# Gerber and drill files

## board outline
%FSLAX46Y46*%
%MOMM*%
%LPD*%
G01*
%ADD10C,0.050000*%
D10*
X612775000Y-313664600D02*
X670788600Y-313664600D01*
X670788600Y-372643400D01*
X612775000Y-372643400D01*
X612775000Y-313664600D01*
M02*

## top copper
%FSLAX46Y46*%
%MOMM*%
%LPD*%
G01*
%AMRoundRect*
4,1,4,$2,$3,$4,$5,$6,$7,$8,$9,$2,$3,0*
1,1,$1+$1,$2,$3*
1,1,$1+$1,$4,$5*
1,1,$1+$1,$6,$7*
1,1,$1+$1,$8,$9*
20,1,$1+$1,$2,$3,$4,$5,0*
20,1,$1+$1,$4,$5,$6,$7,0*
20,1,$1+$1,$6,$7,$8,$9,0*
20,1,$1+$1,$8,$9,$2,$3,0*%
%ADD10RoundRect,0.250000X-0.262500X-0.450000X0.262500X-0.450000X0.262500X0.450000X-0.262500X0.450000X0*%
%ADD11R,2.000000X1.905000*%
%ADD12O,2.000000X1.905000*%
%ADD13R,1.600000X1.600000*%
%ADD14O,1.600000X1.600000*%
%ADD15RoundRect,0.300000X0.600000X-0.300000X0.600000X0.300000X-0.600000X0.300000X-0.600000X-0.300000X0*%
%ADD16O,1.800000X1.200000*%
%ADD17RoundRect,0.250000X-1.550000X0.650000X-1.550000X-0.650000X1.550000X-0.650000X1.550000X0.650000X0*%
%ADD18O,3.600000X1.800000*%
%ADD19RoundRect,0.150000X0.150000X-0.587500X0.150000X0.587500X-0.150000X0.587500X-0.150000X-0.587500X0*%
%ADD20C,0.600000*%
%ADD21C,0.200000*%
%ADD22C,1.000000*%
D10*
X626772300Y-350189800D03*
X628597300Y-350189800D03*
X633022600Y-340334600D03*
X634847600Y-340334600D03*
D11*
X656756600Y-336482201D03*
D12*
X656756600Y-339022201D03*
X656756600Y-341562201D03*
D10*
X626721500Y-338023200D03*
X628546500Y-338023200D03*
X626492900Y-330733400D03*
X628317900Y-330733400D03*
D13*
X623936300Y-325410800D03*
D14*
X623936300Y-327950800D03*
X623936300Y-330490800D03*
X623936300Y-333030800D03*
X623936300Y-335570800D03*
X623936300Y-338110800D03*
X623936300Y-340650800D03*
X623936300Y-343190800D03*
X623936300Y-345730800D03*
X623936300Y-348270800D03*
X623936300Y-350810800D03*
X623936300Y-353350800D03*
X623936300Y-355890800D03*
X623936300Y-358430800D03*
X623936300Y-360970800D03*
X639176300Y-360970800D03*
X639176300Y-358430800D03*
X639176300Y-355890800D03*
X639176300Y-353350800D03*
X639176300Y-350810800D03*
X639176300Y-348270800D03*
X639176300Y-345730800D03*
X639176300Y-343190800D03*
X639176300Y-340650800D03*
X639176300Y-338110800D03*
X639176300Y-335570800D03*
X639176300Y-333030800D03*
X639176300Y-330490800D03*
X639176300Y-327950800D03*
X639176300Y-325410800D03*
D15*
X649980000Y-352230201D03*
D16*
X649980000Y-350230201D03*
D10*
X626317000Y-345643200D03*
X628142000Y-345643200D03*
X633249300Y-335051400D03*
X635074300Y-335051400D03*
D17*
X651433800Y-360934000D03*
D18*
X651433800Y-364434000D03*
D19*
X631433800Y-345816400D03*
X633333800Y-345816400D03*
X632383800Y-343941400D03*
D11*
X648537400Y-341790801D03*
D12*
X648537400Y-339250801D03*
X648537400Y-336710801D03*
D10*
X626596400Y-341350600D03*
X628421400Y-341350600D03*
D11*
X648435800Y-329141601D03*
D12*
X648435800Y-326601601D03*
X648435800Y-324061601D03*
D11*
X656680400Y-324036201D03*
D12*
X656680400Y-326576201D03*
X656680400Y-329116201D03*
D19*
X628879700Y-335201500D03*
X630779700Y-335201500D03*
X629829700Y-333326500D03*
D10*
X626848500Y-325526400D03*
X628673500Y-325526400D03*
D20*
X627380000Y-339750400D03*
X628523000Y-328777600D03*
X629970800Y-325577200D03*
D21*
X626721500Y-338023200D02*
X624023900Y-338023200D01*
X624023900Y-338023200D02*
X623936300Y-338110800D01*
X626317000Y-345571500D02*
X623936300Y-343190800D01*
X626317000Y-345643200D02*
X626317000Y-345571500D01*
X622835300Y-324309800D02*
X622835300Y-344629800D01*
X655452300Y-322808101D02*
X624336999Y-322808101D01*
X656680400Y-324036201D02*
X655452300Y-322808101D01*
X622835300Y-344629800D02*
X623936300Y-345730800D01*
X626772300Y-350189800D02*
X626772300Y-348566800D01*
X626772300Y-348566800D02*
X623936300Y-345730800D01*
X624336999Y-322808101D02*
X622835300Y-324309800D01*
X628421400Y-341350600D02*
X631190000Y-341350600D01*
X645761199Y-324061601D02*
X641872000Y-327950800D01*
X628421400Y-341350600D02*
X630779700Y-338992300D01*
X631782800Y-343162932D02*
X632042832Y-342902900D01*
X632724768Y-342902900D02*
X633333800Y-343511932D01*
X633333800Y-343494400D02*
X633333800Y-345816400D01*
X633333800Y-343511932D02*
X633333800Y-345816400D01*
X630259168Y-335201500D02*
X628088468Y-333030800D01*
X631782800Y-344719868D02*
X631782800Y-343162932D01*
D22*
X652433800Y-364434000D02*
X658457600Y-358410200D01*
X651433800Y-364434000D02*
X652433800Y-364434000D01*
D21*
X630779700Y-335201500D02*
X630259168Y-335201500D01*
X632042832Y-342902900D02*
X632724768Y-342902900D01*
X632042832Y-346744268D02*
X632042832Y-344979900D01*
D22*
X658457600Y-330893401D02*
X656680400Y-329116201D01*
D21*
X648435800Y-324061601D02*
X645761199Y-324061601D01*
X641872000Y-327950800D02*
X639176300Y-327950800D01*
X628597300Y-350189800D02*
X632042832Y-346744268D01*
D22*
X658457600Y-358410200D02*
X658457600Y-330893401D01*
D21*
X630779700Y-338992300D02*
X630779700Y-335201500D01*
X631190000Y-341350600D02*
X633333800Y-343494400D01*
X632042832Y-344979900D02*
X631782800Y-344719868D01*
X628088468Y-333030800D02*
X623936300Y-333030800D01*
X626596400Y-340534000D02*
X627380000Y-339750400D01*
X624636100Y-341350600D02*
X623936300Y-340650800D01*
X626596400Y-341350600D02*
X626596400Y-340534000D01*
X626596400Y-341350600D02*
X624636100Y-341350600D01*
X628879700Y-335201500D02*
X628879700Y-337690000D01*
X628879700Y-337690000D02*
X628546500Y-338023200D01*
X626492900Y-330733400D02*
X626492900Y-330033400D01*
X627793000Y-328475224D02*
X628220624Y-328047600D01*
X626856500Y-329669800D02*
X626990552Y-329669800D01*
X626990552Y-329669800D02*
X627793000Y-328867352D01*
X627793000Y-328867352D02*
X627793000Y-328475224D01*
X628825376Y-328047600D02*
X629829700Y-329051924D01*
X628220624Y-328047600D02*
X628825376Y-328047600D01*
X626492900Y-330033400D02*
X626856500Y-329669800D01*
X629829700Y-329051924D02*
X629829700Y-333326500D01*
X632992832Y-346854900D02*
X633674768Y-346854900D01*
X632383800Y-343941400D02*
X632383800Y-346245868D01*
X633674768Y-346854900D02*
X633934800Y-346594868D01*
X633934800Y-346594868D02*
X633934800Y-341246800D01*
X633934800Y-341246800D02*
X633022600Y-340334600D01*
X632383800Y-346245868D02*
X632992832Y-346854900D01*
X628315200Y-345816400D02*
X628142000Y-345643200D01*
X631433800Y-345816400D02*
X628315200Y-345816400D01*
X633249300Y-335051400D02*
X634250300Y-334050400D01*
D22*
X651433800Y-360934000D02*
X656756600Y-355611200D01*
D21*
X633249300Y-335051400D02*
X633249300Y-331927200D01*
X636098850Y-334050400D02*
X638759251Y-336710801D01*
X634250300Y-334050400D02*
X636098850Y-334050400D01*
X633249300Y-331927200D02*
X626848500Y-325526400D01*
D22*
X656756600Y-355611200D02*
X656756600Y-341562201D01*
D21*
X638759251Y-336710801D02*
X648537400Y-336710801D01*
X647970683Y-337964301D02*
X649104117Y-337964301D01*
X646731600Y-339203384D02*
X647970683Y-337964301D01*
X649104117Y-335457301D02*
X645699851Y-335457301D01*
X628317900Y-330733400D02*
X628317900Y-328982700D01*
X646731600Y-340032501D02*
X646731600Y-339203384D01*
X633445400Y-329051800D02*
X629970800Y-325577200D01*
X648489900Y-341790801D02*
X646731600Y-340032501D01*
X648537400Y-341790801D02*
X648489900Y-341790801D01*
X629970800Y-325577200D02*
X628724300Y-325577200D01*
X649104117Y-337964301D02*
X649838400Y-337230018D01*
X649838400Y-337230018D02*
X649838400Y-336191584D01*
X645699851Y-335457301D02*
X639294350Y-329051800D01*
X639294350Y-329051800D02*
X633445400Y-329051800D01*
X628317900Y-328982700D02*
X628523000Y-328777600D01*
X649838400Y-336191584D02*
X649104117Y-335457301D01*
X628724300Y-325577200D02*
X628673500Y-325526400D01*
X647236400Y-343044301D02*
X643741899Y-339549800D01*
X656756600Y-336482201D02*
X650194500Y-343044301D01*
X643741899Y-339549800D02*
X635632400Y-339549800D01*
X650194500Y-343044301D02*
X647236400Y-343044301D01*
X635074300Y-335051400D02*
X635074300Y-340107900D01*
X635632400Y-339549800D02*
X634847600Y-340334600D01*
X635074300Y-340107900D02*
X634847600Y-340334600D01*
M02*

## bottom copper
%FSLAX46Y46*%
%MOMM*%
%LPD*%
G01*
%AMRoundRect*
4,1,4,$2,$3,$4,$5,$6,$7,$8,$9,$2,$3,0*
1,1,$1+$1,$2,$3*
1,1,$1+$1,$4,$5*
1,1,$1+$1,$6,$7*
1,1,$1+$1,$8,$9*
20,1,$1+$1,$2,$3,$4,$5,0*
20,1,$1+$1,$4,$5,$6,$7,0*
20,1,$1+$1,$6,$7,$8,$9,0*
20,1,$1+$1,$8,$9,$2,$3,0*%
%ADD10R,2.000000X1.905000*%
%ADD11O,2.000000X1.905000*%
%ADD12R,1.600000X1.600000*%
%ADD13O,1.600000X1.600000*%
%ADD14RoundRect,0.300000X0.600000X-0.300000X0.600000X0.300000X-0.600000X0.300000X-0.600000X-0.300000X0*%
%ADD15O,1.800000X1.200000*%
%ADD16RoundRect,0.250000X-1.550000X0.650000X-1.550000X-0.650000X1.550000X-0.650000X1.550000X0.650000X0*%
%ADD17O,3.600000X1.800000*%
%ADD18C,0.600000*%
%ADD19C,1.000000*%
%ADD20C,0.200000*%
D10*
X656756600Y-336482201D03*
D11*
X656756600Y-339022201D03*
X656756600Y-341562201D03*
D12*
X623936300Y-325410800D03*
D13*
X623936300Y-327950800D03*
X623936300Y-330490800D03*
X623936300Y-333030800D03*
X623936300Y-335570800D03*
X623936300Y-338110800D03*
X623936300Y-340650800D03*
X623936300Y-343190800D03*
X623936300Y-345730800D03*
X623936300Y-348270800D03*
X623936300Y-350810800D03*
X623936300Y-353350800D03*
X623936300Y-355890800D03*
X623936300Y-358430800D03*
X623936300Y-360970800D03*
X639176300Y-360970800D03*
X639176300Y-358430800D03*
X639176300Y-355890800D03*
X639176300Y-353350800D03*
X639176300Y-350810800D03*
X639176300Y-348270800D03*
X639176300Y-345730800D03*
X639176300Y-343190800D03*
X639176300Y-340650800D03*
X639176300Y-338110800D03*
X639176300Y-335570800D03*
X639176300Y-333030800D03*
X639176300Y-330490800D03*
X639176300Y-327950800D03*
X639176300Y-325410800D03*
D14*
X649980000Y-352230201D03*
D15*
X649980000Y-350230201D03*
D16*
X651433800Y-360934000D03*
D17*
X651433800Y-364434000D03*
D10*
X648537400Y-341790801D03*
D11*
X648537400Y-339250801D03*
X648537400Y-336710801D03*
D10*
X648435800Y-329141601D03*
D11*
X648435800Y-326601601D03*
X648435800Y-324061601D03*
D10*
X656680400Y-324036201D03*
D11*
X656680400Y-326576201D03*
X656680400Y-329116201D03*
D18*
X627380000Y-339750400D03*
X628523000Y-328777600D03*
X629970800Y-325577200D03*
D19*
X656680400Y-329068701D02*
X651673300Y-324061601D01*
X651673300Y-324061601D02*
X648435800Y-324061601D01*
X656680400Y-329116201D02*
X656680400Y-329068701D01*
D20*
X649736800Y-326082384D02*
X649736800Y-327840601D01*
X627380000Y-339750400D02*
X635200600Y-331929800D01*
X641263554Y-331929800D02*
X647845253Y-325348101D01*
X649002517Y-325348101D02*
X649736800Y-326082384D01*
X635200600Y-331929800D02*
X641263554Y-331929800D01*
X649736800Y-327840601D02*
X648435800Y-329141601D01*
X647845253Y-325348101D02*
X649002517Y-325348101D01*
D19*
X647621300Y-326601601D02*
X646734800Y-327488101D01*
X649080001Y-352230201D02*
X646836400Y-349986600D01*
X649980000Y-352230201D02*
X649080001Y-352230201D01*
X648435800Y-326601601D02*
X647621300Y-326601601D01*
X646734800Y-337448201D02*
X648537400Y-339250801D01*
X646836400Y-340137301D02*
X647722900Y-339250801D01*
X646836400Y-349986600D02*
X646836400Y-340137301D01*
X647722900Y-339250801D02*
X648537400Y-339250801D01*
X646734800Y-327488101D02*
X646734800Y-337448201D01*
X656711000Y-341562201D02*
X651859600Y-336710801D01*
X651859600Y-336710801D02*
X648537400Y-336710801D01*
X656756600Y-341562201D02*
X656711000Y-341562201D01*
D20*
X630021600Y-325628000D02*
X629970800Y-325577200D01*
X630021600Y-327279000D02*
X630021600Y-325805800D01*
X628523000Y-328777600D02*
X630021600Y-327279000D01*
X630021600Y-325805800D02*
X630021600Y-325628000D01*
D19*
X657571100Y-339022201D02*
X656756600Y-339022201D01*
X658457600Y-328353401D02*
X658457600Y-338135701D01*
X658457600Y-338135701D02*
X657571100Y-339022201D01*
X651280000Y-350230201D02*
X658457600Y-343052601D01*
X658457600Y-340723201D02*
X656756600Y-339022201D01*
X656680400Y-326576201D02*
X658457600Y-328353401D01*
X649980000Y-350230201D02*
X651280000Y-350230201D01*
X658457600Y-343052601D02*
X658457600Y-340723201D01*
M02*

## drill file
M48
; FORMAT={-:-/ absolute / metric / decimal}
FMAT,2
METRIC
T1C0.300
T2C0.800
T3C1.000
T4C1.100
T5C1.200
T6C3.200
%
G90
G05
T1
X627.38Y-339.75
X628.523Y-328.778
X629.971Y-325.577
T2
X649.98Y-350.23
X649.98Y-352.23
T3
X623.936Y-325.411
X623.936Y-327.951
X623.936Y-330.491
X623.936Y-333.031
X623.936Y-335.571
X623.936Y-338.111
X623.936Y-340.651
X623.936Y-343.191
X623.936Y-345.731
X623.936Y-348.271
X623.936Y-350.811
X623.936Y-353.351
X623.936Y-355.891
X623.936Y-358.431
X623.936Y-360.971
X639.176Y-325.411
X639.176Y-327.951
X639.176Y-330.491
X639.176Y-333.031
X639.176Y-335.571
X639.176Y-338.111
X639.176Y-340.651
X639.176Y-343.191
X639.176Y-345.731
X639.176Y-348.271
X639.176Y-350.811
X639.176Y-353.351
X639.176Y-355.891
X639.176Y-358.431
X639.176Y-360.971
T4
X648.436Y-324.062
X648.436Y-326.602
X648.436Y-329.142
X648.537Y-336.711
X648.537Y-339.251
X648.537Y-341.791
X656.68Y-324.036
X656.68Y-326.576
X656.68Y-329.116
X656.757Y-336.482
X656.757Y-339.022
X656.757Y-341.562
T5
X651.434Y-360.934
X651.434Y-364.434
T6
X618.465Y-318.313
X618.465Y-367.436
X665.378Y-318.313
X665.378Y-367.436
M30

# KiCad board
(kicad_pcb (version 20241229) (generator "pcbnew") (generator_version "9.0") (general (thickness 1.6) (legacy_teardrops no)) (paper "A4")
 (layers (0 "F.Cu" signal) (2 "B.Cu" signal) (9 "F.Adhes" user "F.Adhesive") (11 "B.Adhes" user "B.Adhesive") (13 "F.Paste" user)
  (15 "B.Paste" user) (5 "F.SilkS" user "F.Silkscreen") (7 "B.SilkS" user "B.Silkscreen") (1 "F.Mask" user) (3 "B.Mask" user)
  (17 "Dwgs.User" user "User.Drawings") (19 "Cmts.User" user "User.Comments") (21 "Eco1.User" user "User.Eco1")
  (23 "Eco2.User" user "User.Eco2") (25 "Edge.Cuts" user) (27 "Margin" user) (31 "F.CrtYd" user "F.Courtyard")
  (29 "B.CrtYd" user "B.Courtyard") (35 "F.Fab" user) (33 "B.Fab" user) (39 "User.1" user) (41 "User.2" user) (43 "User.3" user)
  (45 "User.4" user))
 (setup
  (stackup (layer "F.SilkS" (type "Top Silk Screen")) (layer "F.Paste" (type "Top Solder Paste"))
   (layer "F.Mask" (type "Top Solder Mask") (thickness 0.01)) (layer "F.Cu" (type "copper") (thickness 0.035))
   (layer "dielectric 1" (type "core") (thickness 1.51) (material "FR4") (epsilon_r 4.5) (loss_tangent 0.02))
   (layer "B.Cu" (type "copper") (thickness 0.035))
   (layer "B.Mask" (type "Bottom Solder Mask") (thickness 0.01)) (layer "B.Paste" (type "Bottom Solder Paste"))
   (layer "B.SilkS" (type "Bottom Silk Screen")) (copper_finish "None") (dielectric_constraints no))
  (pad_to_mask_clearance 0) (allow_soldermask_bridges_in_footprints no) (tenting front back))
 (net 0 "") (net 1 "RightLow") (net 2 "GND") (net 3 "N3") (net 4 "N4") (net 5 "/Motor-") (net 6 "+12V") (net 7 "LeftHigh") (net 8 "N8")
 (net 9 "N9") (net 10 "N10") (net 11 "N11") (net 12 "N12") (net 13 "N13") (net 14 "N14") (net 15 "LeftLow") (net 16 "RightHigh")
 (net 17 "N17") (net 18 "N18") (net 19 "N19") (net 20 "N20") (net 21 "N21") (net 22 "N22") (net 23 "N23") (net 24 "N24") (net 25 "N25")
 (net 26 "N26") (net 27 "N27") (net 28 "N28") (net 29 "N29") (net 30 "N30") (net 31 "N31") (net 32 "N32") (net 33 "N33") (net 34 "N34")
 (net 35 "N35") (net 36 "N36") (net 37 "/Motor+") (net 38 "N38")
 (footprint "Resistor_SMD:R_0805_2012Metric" (layer "F.Cu") (at 627.6848 350.1898)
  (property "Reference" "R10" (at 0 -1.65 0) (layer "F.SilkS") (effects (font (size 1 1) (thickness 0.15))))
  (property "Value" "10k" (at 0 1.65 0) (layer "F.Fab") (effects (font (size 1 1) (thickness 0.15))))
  (pad "1" smd roundrect (at -0.9125 0) (size 1.025 1.4) (layers "F.Cu" "F.Mask" "F.Paste") (roundrect_rratio 0.243902) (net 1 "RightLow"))
  (pad "2" smd roundrect (at 0.9125 0) (size 1.025 1.4) (layers "F.Cu" "F.Mask" "F.Paste") (roundrect_rratio 0.243902) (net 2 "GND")))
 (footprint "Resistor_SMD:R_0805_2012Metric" (layer "F.Cu") (at 633.9351 340.3346)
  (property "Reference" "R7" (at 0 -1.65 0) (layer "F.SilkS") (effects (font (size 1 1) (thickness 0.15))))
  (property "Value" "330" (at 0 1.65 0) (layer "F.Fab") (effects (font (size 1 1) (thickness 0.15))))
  (pad "1" smd roundrect (at -0.9125 0) (size 1.025 1.4) (layers "F.Cu" "F.Mask" "F.Paste") (roundrect_rratio 0.243902) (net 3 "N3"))
  (pad "2" smd roundrect (at 0.9125 0) (size 1.025 1.4) (layers "F.Cu" "F.Mask" "F.Paste") (roundrect_rratio 0.243902) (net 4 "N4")))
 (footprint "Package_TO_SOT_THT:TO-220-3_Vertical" (layer "F.Cu") (at 656.7566 336.482201 -90)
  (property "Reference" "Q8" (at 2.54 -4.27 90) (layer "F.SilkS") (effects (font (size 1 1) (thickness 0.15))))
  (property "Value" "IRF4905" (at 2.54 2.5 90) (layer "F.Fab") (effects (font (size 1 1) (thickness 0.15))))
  (pad "1" thru_hole rect (at 0 0 270) (size 1.905 2) (drill 1.1) (layers "*.Cu" "*.Mask") (remove_unused_layers no) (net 4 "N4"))
  (pad "2" thru_hole oval (at 2.54 0 270) (size 1.905 2) (drill 1.1) (layers "*.Cu" "*.Mask") (remove_unused_layers no) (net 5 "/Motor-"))
  (pad "3" thru_hole oval (at 5.08 0 270) (size 1.905 2) (drill 1.1) (layers "*.Cu" "*.Mask") (remove_unused_layers no) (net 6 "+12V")))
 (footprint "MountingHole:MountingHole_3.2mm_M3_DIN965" (layer "F.Cu") (at 665.3784 318.3128)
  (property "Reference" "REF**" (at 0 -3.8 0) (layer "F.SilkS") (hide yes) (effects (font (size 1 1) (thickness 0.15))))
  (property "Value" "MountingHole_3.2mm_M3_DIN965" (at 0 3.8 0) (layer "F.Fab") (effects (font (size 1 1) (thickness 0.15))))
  (pad "" np_thru_hole circle (at 0 0) (size 3.2 3.2) (drill 3.2) (layers "*.Cu" "*.Mask")))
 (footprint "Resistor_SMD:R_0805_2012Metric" (layer "F.Cu") (at 627.634 338.0232)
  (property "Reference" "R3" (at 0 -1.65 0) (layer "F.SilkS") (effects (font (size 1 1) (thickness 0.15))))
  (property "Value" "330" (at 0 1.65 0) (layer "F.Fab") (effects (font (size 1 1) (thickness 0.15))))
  (pad "1" smd roundrect (at -0.9125 0) (size 1.025 1.4) (layers "F.Cu" "F.Mask" "F.Paste") (roundrect_rratio 0.243902) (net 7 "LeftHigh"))
  (pad "2" smd roundrect (at 0.9125 0) (size 1.025 1.4) (layers "F.Cu" "F.Mask" "F.Paste") (roundrect_rratio 0.243902) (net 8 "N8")))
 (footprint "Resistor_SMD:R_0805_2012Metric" (layer "F.Cu") (at 627.4054 330.7334)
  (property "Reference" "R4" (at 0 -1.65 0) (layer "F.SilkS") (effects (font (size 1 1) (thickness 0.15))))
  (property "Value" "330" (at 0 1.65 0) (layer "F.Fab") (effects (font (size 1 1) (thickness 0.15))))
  (pad "1" smd roundrect (at -0.9125 0) (size 1.025 1.4) (layers "F.Cu" "F.Mask" "F.Paste") (roundrect_rratio 0.243902) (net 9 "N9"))
  (pad "2" smd roundrect (at 0.9125 0) (size 1.025 1.4) (layers "F.Cu" "F.Mask" "F.Paste") (roundrect_rratio 0.243902) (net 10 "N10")))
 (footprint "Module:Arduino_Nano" (layer "F.Cu") (at 623.9363 325.4108)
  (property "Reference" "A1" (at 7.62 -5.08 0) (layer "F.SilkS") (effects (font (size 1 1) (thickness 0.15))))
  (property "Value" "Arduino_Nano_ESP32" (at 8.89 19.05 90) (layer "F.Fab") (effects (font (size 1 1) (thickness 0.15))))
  (pad "1" thru_hole rect (at 0 0) (size 1.6 1.6) (drill 1) (layers "*.Cu" "*.Mask") (remove_unused_layers no) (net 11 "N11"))
  (pad "2" thru_hole oval (at 0 2.54) (size 1.6 1.6) (drill 1) (layers "*.Cu" "*.Mask") (remove_unused_layers no) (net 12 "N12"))
  (pad "3" thru_hole oval (at 0 5.08) (size 1.6 1.6) (drill 1) (layers "*.Cu" "*.Mask") (remove_unused_layers no) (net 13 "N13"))
  (pad "4" thru_hole oval (at 0 7.62) (size 1.6 1.6) (drill 1) (layers "*.Cu" "*.Mask") (remove_unused_layers no) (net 2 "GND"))
  (pad "5" thru_hole oval (at 0 10.16) (size 1.6 1.6) (drill 1) (layers "*.Cu" "*.Mask") (remove_unused_layers no) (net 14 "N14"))
  (pad "6" thru_hole oval (at 0 12.7) (size 1.6 1.6) (drill 1) (layers "*.Cu" "*.Mask") (remove_unused_layers no) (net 7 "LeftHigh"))
  (pad "7" thru_hole oval (at 0 15.24) (size 1.6 1.6) (drill 1) (layers "*.Cu" "*.Mask") (remove_unused_layers no) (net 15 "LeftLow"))
  (pad "8" thru_hole oval (at 0 17.78) (size 1.6 1.6) (drill 1) (layers "*.Cu" "*.Mask") (remove_unused_layers no) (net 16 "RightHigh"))
  (pad "9" thru_hole oval (at 0 20.32) (size 1.6 1.6) (drill 1) (layers "*.Cu" "*.Mask") (remove_unused_layers no) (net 1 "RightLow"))
  (pad "10" thru_hole oval (at 0 22.86) (size 1.6 1.6) (drill 1) (layers "*.Cu" "*.Mask") (remove_unused_layers no) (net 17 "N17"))
  (pad "11" thru_hole oval (at 0 25.4) (size 1.6 1.6) (drill 1) (layers "*.Cu" "*.Mask") (remove_unused_layers no) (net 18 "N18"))
  (pad "12" thru_hole oval (at 0 27.94) (size 1.6 1.6) (drill 1) (layers "*.Cu" "*.Mask") (remove_unused_layers no) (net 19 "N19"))
  (pad "13" thru_hole oval (at 0 30.48) (size 1.6 1.6) (drill 1) (layers "*.Cu" "*.Mask") (remove_unused_layers no) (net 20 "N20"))
  (pad "14" thru_hole oval (at 0 33.02) (size 1.6 1.6) (drill 1) (layers "*.Cu" "*.Mask") (remove_unused_layers no) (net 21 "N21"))
  (pad "15" thru_hole oval (at 0 35.56) (size 1.6 1.6) (drill 1) (layers "*.Cu" "*.Mask") (remove_unused_layers no) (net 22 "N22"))
  (pad "16" thru_hole oval (at 15.24 35.56) (size 1.6 1.6) (drill 1) (layers "*.Cu" "*.Mask") (remove_unused_layers no) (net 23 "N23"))
  (pad "17" thru_hole oval (at 15.24 33.02) (size 1.6 1.6) (drill 1) (layers "*.Cu" "*.Mask") (remove_unused_layers no) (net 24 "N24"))
  (pad "18" thru_hole oval (at 15.24 30.48) (size 1.6 1.6) (drill 1) (layers "*.Cu" "*.Mask") (remove_unused_layers no) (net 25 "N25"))
  (pad "19" thru_hole oval (at 15.24 27.94) (size 1.6 1.6) (drill 1) (layers "*.Cu" "*.Mask") (remove_unused_layers no) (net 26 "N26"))
  (pad "20" thru_hole oval (at 15.24 25.4) (size 1.6 1.6) (drill 1) (layers "*.Cu" "*.Mask") (remove_unused_layers no) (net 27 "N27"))
  (pad "21" thru_hole oval (at 15.24 22.86) (size 1.6 1.6) (drill 1) (layers "*.Cu" "*.Mask") (remove_unused_layers no) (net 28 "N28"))
  (pad "22" thru_hole oval (at 15.24 20.32) (size 1.6 1.6) (drill 1) (layers "*.Cu" "*.Mask") (remove_unused_layers no) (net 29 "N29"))
  (pad "23" thru_hole oval (at 15.24 17.78) (size 1.6 1.6) (drill 1) (layers "*.Cu" "*.Mask") (remove_unused_layers no) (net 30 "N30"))
  (pad "24" thru_hole oval (at 15.24 15.24) (size 1.6 1.6) (drill 1) (layers "*.Cu" "*.Mask") (remove_unused_layers no) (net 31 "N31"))
  (pad "25" thru_hole oval (at 15.24 12.7) (size 1.6 1.6) (drill 1) (layers "*.Cu" "*.Mask") (remove_unused_layers no) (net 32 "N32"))
  (pad "26" thru_hole oval (at 15.24 10.16) (size 1.6 1.6) (drill 1) (layers "*.Cu" "*.Mask") (remove_unused_layers no) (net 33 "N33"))
  (pad "27" thru_hole oval (at 15.24 7.62) (size 1.6 1.6) (drill 1) (layers "*.Cu" "*.Mask") (remove_unused_layers no) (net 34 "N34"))
  (pad "28" thru_hole oval (at 15.24 5.08) (size 1.6 1.6) (drill 1) (layers "*.Cu" "*.Mask") (remove_unused_layers no) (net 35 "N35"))
  (pad "29" thru_hole oval (at 15.24 2.54) (size 1.6 1.6) (drill 1) (layers "*.Cu" "*.Mask") (remove_unused_layers no) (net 2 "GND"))
  (pad "30" thru_hole oval (at 15.24 0) (size 1.6 1.6) (drill 1) (layers "*.Cu" "*.Mask") (remove_unused_layers no) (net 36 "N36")))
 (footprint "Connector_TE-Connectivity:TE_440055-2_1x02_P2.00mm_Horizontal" (layer "F.Cu") (at 649.98 352.230201 90)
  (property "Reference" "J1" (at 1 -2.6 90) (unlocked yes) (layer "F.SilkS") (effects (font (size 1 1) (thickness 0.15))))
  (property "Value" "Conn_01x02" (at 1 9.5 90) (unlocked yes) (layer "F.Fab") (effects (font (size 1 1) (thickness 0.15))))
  (pad "1" thru_hole roundrect (at 0 0 90) (size 1.2 1.8) (drill 0.8) (layers "*.Cu" "*.Mask") (remove_unused_layers no)
   (roundrect_rratio 0.25) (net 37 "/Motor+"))
  (pad "2" thru_hole oval (at 2 0 90) (size 1.2 1.8) (drill 0.8) (layers "*.Cu" "*.Mask") (remove_unused_layers no) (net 5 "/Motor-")))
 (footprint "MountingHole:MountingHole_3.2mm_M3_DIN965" (layer "F.Cu") (at 618.4646 367.4364)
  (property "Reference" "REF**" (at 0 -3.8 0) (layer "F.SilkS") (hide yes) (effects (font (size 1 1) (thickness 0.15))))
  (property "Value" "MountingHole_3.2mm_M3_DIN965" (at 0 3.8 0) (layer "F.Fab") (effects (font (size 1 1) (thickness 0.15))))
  (pad "" np_thru_hole circle (at 0 0) (size 3.2 3.2) (drill 3.2) (layers "*.Cu" "*.Mask")))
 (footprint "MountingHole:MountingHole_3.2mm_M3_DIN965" (layer "F.Cu") (at 618.4646 318.3128)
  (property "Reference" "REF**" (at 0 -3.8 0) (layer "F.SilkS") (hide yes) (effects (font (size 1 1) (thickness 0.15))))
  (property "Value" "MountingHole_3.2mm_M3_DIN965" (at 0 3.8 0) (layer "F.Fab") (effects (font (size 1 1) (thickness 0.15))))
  (pad "" np_thru_hole circle (at 0 0) (size 3.2 3.2) (drill 3.2) (layers "*.Cu" "*.Mask")))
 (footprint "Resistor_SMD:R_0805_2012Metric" (layer "F.Cu") (at 627.2295 345.6432)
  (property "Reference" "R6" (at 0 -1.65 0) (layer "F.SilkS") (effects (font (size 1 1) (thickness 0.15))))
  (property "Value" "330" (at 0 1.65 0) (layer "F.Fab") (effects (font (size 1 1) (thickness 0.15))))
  (pad "1" smd roundrect (at -0.9125 0) (size 1.025 1.4) (layers "F.Cu" "F.Mask" "F.Paste") (roundrect_rratio 0.243902) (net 16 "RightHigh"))
  (pad "2" smd roundrect (at 0.9125 0) (size 1.025 1.4) (layers "F.Cu" "F.Mask" "F.Paste") (roundrect_rratio 0.243902) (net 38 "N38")))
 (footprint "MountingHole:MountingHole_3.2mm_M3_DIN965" (layer "F.Cu") (at 665.3784 367.4364)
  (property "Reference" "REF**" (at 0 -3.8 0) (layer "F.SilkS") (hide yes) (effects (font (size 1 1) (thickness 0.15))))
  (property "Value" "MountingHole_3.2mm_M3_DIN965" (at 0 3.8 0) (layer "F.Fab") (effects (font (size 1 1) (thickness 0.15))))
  (pad "" np_thru_hole circle (at 0 0) (size 3.2 3.2) (drill 3.2) (layers "*.Cu" "*.Mask")))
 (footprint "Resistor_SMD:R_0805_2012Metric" (layer "F.Cu") (at 634.1618 335.0514)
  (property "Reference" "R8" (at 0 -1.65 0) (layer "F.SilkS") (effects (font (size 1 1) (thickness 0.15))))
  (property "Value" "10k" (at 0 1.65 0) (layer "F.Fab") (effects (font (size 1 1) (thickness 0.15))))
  (pad "1" smd roundrect (at -0.9125 0) (size 1.025 1.4) (layers "F.Cu" "F.Mask" "F.Paste") (roundrect_rratio 0.243902) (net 6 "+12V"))
  (pad "2" smd roundrect (at 0.9125 0) (size 1.025 1.4) (layers "F.Cu" "F.Mask" "F.Paste") (roundrect_rratio 0.243902) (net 4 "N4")))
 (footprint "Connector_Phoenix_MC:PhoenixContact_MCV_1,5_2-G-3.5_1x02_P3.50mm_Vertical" (layer "F.Cu") (at 651.4338 360.934 -90)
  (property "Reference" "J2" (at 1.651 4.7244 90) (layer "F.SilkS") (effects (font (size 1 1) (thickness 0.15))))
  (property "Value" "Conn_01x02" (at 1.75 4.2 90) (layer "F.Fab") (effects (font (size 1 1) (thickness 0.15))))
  (pad "1" thru_hole roundrect (at 0 0 270) (size 1.8 3.6) (drill 1.2) (layers "*.Cu" "*.Mask") (remove_unused_layers no)
   (roundrect_rratio 0.138889) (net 6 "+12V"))
  (pad "2" thru_hole oval (at 3.5 0 270) (size 1.8 3.6) (drill 1.2) (layers "*.Cu" "*.Mask") (remove_unused_layers no) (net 2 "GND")))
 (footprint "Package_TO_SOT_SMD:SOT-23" (layer "F.Cu") (at 632.3838 344.8789 90)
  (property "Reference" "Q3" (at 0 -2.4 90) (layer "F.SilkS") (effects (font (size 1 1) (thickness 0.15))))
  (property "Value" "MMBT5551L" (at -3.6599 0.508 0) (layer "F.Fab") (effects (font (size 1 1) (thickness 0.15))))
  (pad "1" smd roundrect (at -0.9375 -0.95 90) (size 1.475 0.6) (layers "F.Cu" "F.Mask" "F.Paste") (roundrect_rratio 0.25) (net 38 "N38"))
  (pad "2" smd roundrect (at -0.9375 0.95 90) (size 1.475 0.6) (layers "F.Cu" "F.Mask" "F.Paste") (roundrect_rratio 0.25) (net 2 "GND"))
  (pad "3" smd roundrect (at 0.9375 0 90) (size 1.475 0.6) (layers "F.Cu" "F.Mask" "F.Paste") (roundrect_rratio 0.25) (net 3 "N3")))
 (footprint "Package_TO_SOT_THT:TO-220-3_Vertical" (layer "F.Cu") (at 648.5374 341.790801 90)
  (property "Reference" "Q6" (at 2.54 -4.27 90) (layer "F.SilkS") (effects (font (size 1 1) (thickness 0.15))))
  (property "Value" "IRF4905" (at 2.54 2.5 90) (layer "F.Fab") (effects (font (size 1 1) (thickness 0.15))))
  (pad "1" thru_hole rect (at 0 0 90) (size 1.905 2) (drill 1.1) (layers "*.Cu" "*.Mask") (remove_unused_layers no) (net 10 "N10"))
  (pad "2" thru_hole oval (at 2.54 0 90) (size 1.905 2) (drill 1.1) (layers "*.Cu" "*.Mask") (remove_unused_layers no) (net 37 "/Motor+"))
  (pad "3" thru_hole oval (at 5.08 0 90) (size 1.905 2) (drill 1.1) (layers "*.Cu" "*.Mask") (remove_unused_layers no) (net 6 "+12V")))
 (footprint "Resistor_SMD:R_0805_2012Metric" (layer "F.Cu") (at 627.5089 341.3506)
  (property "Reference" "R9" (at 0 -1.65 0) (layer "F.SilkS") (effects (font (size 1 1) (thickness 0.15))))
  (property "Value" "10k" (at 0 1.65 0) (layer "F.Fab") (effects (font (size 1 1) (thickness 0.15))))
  (pad "1" smd roundrect (at -0.9125 0) (size 1.025 1.4) (layers "F.Cu" "F.Mask" "F.Paste") (roundrect_rratio 0.243902) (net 15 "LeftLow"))
  (pad "2" smd roundrect (at 0.9125 0) (size 1.025 1.4) (layers "F.Cu" "F.Mask" "F.Paste") (roundrect_rratio 0.243902) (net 2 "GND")))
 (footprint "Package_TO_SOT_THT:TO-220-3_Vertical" (layer "F.Cu") (at 648.4358 329.141601 90)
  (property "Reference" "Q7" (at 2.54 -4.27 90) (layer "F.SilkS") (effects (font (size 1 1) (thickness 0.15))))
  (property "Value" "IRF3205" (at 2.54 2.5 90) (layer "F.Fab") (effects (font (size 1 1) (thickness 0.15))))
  (pad "1" thru_hole rect (at 0 0 90) (size 1.905 2) (drill 1.1) (layers "*.Cu" "*.Mask") (remove_unused_layers no) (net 15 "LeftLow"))
  (pad "2" thru_hole oval (at 2.54 0 90) (size 1.905 2) (drill 1.1) (layers "*.Cu" "*.Mask") (remove_unused_layers no) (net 37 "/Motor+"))
  (pad "3" thru_hole oval (at 5.08 0 90) (size 1.905 2) (drill 1.1) (layers "*.Cu" "*.Mask") (remove_unused_layers no) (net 2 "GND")))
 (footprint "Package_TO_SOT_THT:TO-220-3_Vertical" (layer "F.Cu") (at 656.6804 324.036201 -90)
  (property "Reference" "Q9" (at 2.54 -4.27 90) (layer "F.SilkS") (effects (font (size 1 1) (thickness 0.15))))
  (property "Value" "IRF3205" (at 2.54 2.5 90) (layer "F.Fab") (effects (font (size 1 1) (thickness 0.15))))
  (pad "1" thru_hole rect (at 0 0 270) (size 1.905 2) (drill 1.1) (layers "*.Cu" "*.Mask") (remove_unused_layers no) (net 1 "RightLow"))
  (pad "2" thru_hole oval (at 2.54 0 270) (size 1.905 2) (drill 1.1) (layers "*.Cu" "*.Mask") (remove_unused_layers no) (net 5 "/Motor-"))
  (pad "3" thru_hole oval (at 5.08 0 270) (size 1.905 2) (drill 1.1) (layers "*.Cu" "*.Mask") (remove_unused_layers no) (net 2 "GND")))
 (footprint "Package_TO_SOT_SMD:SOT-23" (layer "F.Cu") (at 629.8297 334.264 90)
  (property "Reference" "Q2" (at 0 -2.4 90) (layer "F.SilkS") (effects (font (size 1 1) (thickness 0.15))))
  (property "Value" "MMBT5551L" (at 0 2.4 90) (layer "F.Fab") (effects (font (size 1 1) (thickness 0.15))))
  (pad "1" smd roundrect (at -0.9375 -0.95 90) (size 1.475 0.6) (layers "F.Cu" "F.Mask" "F.Paste") (roundrect_rratio 0.25) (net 8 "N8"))
  (pad "2" smd roundrect (at -0.9375 0.95 90) (size 1.475 0.6) (layers "F.Cu" "F.Mask" "F.Paste") (roundrect_rratio 0.25) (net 2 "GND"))
  (pad "3" smd roundrect (at 0.9375 0 90) (size 1.475 0.6) (layers "F.Cu" "F.Mask" "F.Paste") (roundrect_rratio 0.25) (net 9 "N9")))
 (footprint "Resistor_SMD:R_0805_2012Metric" (layer "F.Cu") (at 627.761 325.5264)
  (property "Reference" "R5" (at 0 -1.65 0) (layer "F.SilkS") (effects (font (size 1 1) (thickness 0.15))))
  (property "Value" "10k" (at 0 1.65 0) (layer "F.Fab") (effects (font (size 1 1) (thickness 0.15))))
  (pad "1" smd roundrect (at -0.9125 0) (size 1.025 1.4) (layers "F.Cu" "F.Mask" "F.Paste") (roundrect_rratio 0.243902) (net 6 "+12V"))
  (pad "2" smd roundrect (at 0.9125 0) (size 1.025 1.4) (layers "F.Cu" "F.Mask" "F.Paste") (roundrect_rratio 0.243902) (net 10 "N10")))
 (gr_rect (start 612.775 313.6646) (end 670.7886 372.6434) (stroke (width 0.05) (type default)) (fill no) (layer "Edge.Cuts"))
 (segment (start 626.7215 338.0232) (end 624.0239 338.0232) (width 0.2) (layer "F.Cu") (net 7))
 (segment (start 624.0239 338.0232) (end 623.9363 338.1108) (width 0.2) (layer "F.Cu") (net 7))
 (segment (start 626.317 345.5715) (end 623.9363 343.1908) (width 0.2) (layer "F.Cu") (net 16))
 (segment (start 626.317 345.6432) (end 626.317 345.5715) (width 0.2) (layer "F.Cu") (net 16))
 (segment (start 622.8353 324.3098) (end 622.8353 344.6298) (width 0.2) (layer "F.Cu") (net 1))
 (segment (start 655.4523 322.808101) (end 624.336999 322.808101) (width 0.2) (layer "F.Cu") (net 1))
 (segment (start 656.6804 324.036201) (end 655.4523 322.808101) (width 0.2) (layer "F.Cu") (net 1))
 (segment (start 622.8353 344.6298) (end 623.9363 345.7308) (width 0.2) (layer "F.Cu") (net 1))
 (segment (start 626.7723 350.1898) (end 626.7723 348.5668) (width 0.2) (layer "F.Cu") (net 1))
 (segment (start 626.7723 348.5668) (end 623.9363 345.7308) (width 0.2) (layer "F.Cu") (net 1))
 (segment (start 624.336999 322.808101) (end 622.8353 324.3098) (width 0.2) (layer "F.Cu") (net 1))
 (segment (start 628.4214 341.3506) (end 631.19 341.3506) (width 0.2) (layer "F.Cu") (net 2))
 (segment (start 645.761199 324.061601) (end 641.872 327.9508) (width 0.2) (layer "F.Cu") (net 2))
 (segment (start 628.4214 341.3506) (end 630.7797 338.9923) (width 0.2) (layer "F.Cu") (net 2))
 (segment (start 631.7828 343.162932) (end 632.042832 342.9029) (width 0.2) (layer "F.Cu") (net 2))
 (segment (start 632.724768 342.9029) (end 633.3338 343.511932) (width 0.2) (layer "F.Cu") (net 2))
 (segment (start 633.3338 343.4944) (end 633.3338 345.8164) (width 0.2) (layer "F.Cu") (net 2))
 (segment (start 633.3338 343.511932) (end 633.3338 345.8164) (width 0.2) (layer "F.Cu") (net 2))
 (segment (start 630.259168 335.2015) (end 628.088468 333.0308) (width 0.2) (layer "F.Cu") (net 2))
 (segment (start 631.7828 344.719868) (end 631.7828 343.162932) (width 0.2) (layer "F.Cu") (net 2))
 (segment (start 652.4338 364.434) (end 658.4576 358.4102) (width 1) (layer "F.Cu") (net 2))
 (segment (start 651.4338 364.434) (end 652.4338 364.434) (width 1) (layer "F.Cu") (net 2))
 (segment (start 630.7797 335.2015) (end 630.259168 335.2015) (width 0.2) (layer "F.Cu") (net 2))
 (segment (start 632.042832 342.9029) (end 632.724768 342.9029) (width 0.2) (layer "F.Cu") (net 2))
 (segment (start 632.042832 346.744268) (end 632.042832 344.9799) (width 0.2) (layer "F.Cu") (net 2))
 (segment (start 658.4576 330.893401) (end 656.6804 329.116201) (width 1) (layer "F.Cu") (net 2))
 (segment (start 648.4358 324.061601) (end 645.761199 324.061601) (width 0.2) (layer "F.Cu") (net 2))
 (segment (start 641.872 327.9508) (end 639.1763 327.9508) (width 0.2) (layer "F.Cu") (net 2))
 (segment (start 628.5973 350.1898) (end 632.042832 346.744268) (width 0.2) (layer "F.Cu") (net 2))
 (segment (start 658.4576 358.4102) (end 658.4576 330.893401) (width 1) (layer "F.Cu") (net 2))
 (segment (start 630.7797 338.9923) (end 630.7797 335.2015) (width 0.2) (layer "F.Cu") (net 2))
 (segment (start 631.19 341.3506) (end 633.3338 343.4944) (width 0.2) (layer "F.Cu") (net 2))
 (segment (start 632.042832 344.9799) (end 631.7828 344.719868) (width 0.2) (layer "F.Cu") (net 2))
 (segment (start 628.088468 333.0308) (end 623.9363 333.0308) (width 0.2) (layer "F.Cu") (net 2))
 (segment (start 656.6804 329.068701) (end 651.6733 324.061601) (width 1) (layer "B.Cu") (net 2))
 (segment (start 651.6733 324.061601) (end 648.4358 324.061601) (width 1) (layer "B.Cu") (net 2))
 (segment (start 656.6804 329.116201) (end 656.6804 329.068701) (width 1) (layer "B.Cu") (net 2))
 (segment (start 626.5964 340.534) (end 627.38 339.7504) (width 0.2) (layer "F.Cu") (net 15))
 (segment (start 624.6361 341.3506) (end 623.9363 340.6508) (width 0.2) (layer "F.Cu") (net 15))
 (segment (start 626.5964 341.3506) (end 626.5964 340.534) (width 0.2) (layer "F.Cu") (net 15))
 (segment (start 626.5964 341.3506) (end 624.6361 341.3506) (width 0.2) (layer "F.Cu") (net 15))
 (via (at 627.38 339.7504) (size 0.6) (drill 0.3) (layers "F.Cu" "B.Cu") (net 15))
 (segment (start 649.7368 326.082384) (end 649.7368 327.840601) (width 0.2) (layer "B.Cu") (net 15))
 (segment (start 627.38 339.7504) (end 635.2006 331.9298) (width 0.2) (layer "B.Cu") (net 15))
 (segment (start 641.263554 331.9298) (end 647.845253 325.348101) (width 0.2) (layer "B.Cu") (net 15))
 (segment (start 649.002517 325.348101) (end 649.7368 326.082384) (width 0.2) (layer "B.Cu") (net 15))
 (segment (start 635.2006 331.9298) (end 641.263554 331.9298) (width 0.2) (layer "B.Cu") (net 15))
 (segment (start 649.7368 327.840601) (end 648.4358 329.141601) (width 0.2) (layer "B.Cu") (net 15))
 (segment (start 647.845253 325.348101) (end 649.002517 325.348101) (width 0.2) (layer "B.Cu") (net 15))
 (segment (start 628.8797 335.2015) (end 628.8797 337.69) (width 0.2) (layer "F.Cu") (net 8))
 (segment (start 628.8797 337.69) (end 628.5465 338.0232) (width 0.2) (layer "F.Cu") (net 8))
 (segment (start 626.4929 330.7334) (end 626.4929 330.0334) (width 0.2) (layer "F.Cu") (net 9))
 (segment (start 627.793 328.475224) (end 628.220624 328.0476) (width 0.2) (layer "F.Cu") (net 9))
 (segment (start 626.8565 329.6698) (end 626.990552 329.6698) (width 0.2) (layer "F.Cu") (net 9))
 (segment (start 626.990552 329.6698) (end 627.793 328.867352) (width 0.2) (layer "F.Cu") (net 9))
 (segment (start 627.793 328.867352) (end 627.793 328.475224) (width 0.2) (layer "F.Cu") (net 9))
 (segment (start 628.825376 328.0476) (end 629.8297 329.051924) (width 0.2) (layer "F.Cu") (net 9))
 (segment (start 628.220624 328.0476) (end 628.825376 328.0476) (width 0.2) (layer "F.Cu") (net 9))
 (segment (start 626.4929 330.0334) (end 626.8565 329.6698) (width 0.2) (layer "F.Cu") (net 9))
 (segment (start 629.8297 329.051924) (end 629.8297 333.3265) (width 0.2) (layer "F.Cu") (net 9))
 (segment (start 632.992832 346.8549) (end 633.674768 346.8549) (width 0.2) (layer "F.Cu") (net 3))
 (segment (start 632.3838 343.9414) (end 632.3838 346.245868) (width 0.2) (layer "F.Cu") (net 3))
 (segment (start 633.674768 346.8549) (end 633.9348 346.594868) (width 0.2) (layer "F.Cu") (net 3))
 (segment (start 633.9348 346.594868) (end 633.9348 341.2468) (width 0.2) (layer "F.Cu") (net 3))
 (segment (start 633.9348 341.2468) (end 633.0226 340.3346) (width 0.2) (layer "F.Cu") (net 3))
 (segment (start 632.3838 346.245868) (end 632.992832 346.8549) (width 0.2) (layer "F.Cu") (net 3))
 (segment (start 628.3152 345.8164) (end 628.142 345.6432) (width 0.2) (layer "F.Cu") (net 38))
 (segment (start 631.4338 345.8164) (end 628.3152 345.8164) (width 0.2) (layer "F.Cu") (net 38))
 (segment (start 647.6213 326.601601) (end 646.7348 327.488101) (width 1) (layer "B.Cu") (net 37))
 (segment (start 649.080001 352.230201) (end 646.8364 349.9866) (width 1) (layer "B.Cu") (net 37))
 (segment (start 649.98 352.230201) (end 649.080001 352.230201) (width 1) (layer "B.Cu") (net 37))
 (segment (start 648.4358 326.601601) (end 647.6213 326.601601) (width 1) (layer "B.Cu") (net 37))
 (segment (start 646.7348 337.448201) (end 648.5374 339.250801) (width 1) (layer "B.Cu") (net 37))
 (segment (start 646.8364 340.137301) (end 647.7229 339.250801) (width 1) (layer "B.Cu") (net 37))
 (segment (start 646.8364 349.9866) (end 646.8364 340.137301) (width 1) (layer "B.Cu") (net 37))
 (segment (start 647.7229 339.250801) (end 648.5374 339.250801) (width 1) (layer "B.Cu") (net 37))
 (segment (start 646.7348 327.488101) (end 646.7348 337.448201) (width 1) (layer "B.Cu") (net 37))
 (segment (start 633.2493 335.0514) (end 634.2503 334.0504) (width 0.2) (layer "F.Cu") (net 6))
 (segment (start 651.4338 360.934) (end 656.7566 355.6112) (width 1) (layer "F.Cu") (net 6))
 (segment (start 633.2493 335.0514) (end 633.2493 331.9272) (width 0.2) (layer "F.Cu") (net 6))
 (segment (start 636.09885 334.0504) (end 638.759251 336.710801) (width 0.2) (layer "F.Cu") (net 6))
 (segment (start 634.2503 334.0504) (end 636.09885 334.0504) (width 0.2) (layer "F.Cu") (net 6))
 (segment (start 633.2493 331.9272) (end 626.8485 325.5264) (width 0.2) (layer "F.Cu") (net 6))
 (segment (start 656.7566 355.6112) (end 656.7566 341.562201) (width 1) (layer "F.Cu") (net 6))
 (segment (start 638.759251 336.710801) (end 648.5374 336.710801) (width 0.2) (layer "F.Cu") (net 6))
 (segment (start 656.711 341.562201) (end 651.8596 336.710801) (width 1) (layer "B.Cu") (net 6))
 (segment (start 651.8596 336.710801) (end 648.5374 336.710801) (width 1) (layer "B.Cu") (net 6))
 (segment (start 656.7566 341.562201) (end 656.711 341.562201) (width 1) (layer "B.Cu") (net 6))
 (segment (start 647.970683 337.964301) (end 649.104117 337.964301) (width 0.2) (layer "F.Cu") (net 10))
 (segment (start 646.7316 339.203384) (end 647.970683 337.964301) (width 0.2) (layer "F.Cu") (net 10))
 (segment (start 649.104117 335.457301) (end 645.699851 335.457301) (width 0.2) (layer "F.Cu") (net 10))
 (segment (start 628.3179 330.7334) (end 628.3179 328.9827) (width 0.2) (layer "F.Cu") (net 10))
 (segment (start 646.7316 340.032501) (end 646.7316 339.203384) (width 0.2) (layer "F.Cu") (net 10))
 (segment (start 633.4454 329.0518) (end 629.9708 325.5772) (width 0.2) (layer "F.Cu") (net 10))
 (segment (start 648.4899 341.790801) (end 646.7316 340.032501) (width 0.2) (layer "F.Cu") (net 10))
 (segment (start 648.5374 341.790801) (end 648.4899 341.790801) (width 0.2) (layer "F.Cu") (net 10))
 (segment (start 629.9708 325.5772) (end 628.7243 325.5772) (width 0.2) (layer "F.Cu") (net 10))
 (segment (start 649.104117 337.964301) (end 649.8384 337.230018) (width 0.2) (layer "F.Cu") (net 10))
 (segment (start 649.8384 337.230018) (end 649.8384 336.191584) (width 0.2) (layer "F.Cu") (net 10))
 (segment (start 645.699851 335.457301) (end 639.29435 329.0518) (width 0.2) (layer "F.Cu") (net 10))
 (segment (start 639.29435 329.0518) (end 633.4454 329.0518) (width 0.2) (layer "F.Cu") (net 10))
 (segment (start 628.3179 328.9827) (end 628.523 328.7776) (width 0.2) (layer "F.Cu") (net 10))
 (segment (start 649.8384 336.191584) (end 649.104117 335.457301) (width 0.2) (layer "F.Cu") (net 10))
 (segment (start 628.7243 325.5772) (end 628.6735 325.5264) (width 0.2) (layer "F.Cu") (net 10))
 (via (at 628.523 328.7776) (size 0.6) (drill 0.3) (layers "F.Cu" "B.Cu") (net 10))
 (via (at 629.9708 325.5772) (size 0.6) (drill 0.3) (layers "F.Cu" "B.Cu") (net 10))
 (segment (start 630.0216 325.628) (end 629.9708 325.5772) (width 0.2) (layer "B.Cu") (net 10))
 (segment (start 630.0216 327.279) (end 630.0216 325.8058) (width 0.2) (layer "B.Cu") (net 10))
 (segment (start 628.523 328.7776) (end 630.0216 327.279) (width 0.2) (layer "B.Cu") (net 10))
 (segment (start 630.0216 325.8058) (end 630.0216 325.628) (width 0.2) (layer "B.Cu") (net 10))
 (segment (start 647.2364 343.044301) (end 643.741899 339.5498) (width 0.2) (layer "F.Cu") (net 4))
 (segment (start 656.7566 336.482201) (end 650.1945 343.044301) (width 0.2) (layer "F.Cu") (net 4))
 (segment (start 643.741899 339.5498) (end 635.6324 339.5498) (width 0.2) (layer "F.Cu") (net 4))
 (segment (start 650.1945 343.044301) (end 647.2364 343.044301) (width 0.2) (layer "F.Cu") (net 4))
 (segment (start 635.0743 335.0514) (end 635.0743 340.1079) (width 0.2) (layer "F.Cu") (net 4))
 (segment (start 635.6324 339.5498) (end 634.8476 340.3346) (width 0.2) (layer "F.Cu") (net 4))
 (segment (start 635.0743 340.1079) (end 634.8476 340.3346) (width 0.2) (layer "F.Cu") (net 4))
 (segment (start 657.5711 339.022201) (end 656.7566 339.022201) (width 1) (layer "B.Cu") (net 5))
 (segment (start 658.4576 328.353401) (end 658.4576 338.135701) (width 1) (layer "B.Cu") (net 5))
 (segment (start 658.4576 338.135701) (end 657.5711 339.022201) (width 1) (layer "B.Cu") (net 5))
 (segment (start 651.28 350.230201) (end 658.4576 343.052601) (width 1) (layer "B.Cu") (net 5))
 (segment (start 658.4576 340.723201) (end 656.7566 339.022201) (width 1) (layer "B.Cu") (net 5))
 (segment (start 656.6804 326.576201) (end 658.4576 328.353401) (width 1) (layer "B.Cu") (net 5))
 (segment (start 649.98 350.230201) (end 651.28 350.230201) (width 1) (layer "B.Cu") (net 5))
 (segment (start 658.4576 343.052601) (end 658.4576 340.723201) (width 1) (layer "B.Cu") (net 5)))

